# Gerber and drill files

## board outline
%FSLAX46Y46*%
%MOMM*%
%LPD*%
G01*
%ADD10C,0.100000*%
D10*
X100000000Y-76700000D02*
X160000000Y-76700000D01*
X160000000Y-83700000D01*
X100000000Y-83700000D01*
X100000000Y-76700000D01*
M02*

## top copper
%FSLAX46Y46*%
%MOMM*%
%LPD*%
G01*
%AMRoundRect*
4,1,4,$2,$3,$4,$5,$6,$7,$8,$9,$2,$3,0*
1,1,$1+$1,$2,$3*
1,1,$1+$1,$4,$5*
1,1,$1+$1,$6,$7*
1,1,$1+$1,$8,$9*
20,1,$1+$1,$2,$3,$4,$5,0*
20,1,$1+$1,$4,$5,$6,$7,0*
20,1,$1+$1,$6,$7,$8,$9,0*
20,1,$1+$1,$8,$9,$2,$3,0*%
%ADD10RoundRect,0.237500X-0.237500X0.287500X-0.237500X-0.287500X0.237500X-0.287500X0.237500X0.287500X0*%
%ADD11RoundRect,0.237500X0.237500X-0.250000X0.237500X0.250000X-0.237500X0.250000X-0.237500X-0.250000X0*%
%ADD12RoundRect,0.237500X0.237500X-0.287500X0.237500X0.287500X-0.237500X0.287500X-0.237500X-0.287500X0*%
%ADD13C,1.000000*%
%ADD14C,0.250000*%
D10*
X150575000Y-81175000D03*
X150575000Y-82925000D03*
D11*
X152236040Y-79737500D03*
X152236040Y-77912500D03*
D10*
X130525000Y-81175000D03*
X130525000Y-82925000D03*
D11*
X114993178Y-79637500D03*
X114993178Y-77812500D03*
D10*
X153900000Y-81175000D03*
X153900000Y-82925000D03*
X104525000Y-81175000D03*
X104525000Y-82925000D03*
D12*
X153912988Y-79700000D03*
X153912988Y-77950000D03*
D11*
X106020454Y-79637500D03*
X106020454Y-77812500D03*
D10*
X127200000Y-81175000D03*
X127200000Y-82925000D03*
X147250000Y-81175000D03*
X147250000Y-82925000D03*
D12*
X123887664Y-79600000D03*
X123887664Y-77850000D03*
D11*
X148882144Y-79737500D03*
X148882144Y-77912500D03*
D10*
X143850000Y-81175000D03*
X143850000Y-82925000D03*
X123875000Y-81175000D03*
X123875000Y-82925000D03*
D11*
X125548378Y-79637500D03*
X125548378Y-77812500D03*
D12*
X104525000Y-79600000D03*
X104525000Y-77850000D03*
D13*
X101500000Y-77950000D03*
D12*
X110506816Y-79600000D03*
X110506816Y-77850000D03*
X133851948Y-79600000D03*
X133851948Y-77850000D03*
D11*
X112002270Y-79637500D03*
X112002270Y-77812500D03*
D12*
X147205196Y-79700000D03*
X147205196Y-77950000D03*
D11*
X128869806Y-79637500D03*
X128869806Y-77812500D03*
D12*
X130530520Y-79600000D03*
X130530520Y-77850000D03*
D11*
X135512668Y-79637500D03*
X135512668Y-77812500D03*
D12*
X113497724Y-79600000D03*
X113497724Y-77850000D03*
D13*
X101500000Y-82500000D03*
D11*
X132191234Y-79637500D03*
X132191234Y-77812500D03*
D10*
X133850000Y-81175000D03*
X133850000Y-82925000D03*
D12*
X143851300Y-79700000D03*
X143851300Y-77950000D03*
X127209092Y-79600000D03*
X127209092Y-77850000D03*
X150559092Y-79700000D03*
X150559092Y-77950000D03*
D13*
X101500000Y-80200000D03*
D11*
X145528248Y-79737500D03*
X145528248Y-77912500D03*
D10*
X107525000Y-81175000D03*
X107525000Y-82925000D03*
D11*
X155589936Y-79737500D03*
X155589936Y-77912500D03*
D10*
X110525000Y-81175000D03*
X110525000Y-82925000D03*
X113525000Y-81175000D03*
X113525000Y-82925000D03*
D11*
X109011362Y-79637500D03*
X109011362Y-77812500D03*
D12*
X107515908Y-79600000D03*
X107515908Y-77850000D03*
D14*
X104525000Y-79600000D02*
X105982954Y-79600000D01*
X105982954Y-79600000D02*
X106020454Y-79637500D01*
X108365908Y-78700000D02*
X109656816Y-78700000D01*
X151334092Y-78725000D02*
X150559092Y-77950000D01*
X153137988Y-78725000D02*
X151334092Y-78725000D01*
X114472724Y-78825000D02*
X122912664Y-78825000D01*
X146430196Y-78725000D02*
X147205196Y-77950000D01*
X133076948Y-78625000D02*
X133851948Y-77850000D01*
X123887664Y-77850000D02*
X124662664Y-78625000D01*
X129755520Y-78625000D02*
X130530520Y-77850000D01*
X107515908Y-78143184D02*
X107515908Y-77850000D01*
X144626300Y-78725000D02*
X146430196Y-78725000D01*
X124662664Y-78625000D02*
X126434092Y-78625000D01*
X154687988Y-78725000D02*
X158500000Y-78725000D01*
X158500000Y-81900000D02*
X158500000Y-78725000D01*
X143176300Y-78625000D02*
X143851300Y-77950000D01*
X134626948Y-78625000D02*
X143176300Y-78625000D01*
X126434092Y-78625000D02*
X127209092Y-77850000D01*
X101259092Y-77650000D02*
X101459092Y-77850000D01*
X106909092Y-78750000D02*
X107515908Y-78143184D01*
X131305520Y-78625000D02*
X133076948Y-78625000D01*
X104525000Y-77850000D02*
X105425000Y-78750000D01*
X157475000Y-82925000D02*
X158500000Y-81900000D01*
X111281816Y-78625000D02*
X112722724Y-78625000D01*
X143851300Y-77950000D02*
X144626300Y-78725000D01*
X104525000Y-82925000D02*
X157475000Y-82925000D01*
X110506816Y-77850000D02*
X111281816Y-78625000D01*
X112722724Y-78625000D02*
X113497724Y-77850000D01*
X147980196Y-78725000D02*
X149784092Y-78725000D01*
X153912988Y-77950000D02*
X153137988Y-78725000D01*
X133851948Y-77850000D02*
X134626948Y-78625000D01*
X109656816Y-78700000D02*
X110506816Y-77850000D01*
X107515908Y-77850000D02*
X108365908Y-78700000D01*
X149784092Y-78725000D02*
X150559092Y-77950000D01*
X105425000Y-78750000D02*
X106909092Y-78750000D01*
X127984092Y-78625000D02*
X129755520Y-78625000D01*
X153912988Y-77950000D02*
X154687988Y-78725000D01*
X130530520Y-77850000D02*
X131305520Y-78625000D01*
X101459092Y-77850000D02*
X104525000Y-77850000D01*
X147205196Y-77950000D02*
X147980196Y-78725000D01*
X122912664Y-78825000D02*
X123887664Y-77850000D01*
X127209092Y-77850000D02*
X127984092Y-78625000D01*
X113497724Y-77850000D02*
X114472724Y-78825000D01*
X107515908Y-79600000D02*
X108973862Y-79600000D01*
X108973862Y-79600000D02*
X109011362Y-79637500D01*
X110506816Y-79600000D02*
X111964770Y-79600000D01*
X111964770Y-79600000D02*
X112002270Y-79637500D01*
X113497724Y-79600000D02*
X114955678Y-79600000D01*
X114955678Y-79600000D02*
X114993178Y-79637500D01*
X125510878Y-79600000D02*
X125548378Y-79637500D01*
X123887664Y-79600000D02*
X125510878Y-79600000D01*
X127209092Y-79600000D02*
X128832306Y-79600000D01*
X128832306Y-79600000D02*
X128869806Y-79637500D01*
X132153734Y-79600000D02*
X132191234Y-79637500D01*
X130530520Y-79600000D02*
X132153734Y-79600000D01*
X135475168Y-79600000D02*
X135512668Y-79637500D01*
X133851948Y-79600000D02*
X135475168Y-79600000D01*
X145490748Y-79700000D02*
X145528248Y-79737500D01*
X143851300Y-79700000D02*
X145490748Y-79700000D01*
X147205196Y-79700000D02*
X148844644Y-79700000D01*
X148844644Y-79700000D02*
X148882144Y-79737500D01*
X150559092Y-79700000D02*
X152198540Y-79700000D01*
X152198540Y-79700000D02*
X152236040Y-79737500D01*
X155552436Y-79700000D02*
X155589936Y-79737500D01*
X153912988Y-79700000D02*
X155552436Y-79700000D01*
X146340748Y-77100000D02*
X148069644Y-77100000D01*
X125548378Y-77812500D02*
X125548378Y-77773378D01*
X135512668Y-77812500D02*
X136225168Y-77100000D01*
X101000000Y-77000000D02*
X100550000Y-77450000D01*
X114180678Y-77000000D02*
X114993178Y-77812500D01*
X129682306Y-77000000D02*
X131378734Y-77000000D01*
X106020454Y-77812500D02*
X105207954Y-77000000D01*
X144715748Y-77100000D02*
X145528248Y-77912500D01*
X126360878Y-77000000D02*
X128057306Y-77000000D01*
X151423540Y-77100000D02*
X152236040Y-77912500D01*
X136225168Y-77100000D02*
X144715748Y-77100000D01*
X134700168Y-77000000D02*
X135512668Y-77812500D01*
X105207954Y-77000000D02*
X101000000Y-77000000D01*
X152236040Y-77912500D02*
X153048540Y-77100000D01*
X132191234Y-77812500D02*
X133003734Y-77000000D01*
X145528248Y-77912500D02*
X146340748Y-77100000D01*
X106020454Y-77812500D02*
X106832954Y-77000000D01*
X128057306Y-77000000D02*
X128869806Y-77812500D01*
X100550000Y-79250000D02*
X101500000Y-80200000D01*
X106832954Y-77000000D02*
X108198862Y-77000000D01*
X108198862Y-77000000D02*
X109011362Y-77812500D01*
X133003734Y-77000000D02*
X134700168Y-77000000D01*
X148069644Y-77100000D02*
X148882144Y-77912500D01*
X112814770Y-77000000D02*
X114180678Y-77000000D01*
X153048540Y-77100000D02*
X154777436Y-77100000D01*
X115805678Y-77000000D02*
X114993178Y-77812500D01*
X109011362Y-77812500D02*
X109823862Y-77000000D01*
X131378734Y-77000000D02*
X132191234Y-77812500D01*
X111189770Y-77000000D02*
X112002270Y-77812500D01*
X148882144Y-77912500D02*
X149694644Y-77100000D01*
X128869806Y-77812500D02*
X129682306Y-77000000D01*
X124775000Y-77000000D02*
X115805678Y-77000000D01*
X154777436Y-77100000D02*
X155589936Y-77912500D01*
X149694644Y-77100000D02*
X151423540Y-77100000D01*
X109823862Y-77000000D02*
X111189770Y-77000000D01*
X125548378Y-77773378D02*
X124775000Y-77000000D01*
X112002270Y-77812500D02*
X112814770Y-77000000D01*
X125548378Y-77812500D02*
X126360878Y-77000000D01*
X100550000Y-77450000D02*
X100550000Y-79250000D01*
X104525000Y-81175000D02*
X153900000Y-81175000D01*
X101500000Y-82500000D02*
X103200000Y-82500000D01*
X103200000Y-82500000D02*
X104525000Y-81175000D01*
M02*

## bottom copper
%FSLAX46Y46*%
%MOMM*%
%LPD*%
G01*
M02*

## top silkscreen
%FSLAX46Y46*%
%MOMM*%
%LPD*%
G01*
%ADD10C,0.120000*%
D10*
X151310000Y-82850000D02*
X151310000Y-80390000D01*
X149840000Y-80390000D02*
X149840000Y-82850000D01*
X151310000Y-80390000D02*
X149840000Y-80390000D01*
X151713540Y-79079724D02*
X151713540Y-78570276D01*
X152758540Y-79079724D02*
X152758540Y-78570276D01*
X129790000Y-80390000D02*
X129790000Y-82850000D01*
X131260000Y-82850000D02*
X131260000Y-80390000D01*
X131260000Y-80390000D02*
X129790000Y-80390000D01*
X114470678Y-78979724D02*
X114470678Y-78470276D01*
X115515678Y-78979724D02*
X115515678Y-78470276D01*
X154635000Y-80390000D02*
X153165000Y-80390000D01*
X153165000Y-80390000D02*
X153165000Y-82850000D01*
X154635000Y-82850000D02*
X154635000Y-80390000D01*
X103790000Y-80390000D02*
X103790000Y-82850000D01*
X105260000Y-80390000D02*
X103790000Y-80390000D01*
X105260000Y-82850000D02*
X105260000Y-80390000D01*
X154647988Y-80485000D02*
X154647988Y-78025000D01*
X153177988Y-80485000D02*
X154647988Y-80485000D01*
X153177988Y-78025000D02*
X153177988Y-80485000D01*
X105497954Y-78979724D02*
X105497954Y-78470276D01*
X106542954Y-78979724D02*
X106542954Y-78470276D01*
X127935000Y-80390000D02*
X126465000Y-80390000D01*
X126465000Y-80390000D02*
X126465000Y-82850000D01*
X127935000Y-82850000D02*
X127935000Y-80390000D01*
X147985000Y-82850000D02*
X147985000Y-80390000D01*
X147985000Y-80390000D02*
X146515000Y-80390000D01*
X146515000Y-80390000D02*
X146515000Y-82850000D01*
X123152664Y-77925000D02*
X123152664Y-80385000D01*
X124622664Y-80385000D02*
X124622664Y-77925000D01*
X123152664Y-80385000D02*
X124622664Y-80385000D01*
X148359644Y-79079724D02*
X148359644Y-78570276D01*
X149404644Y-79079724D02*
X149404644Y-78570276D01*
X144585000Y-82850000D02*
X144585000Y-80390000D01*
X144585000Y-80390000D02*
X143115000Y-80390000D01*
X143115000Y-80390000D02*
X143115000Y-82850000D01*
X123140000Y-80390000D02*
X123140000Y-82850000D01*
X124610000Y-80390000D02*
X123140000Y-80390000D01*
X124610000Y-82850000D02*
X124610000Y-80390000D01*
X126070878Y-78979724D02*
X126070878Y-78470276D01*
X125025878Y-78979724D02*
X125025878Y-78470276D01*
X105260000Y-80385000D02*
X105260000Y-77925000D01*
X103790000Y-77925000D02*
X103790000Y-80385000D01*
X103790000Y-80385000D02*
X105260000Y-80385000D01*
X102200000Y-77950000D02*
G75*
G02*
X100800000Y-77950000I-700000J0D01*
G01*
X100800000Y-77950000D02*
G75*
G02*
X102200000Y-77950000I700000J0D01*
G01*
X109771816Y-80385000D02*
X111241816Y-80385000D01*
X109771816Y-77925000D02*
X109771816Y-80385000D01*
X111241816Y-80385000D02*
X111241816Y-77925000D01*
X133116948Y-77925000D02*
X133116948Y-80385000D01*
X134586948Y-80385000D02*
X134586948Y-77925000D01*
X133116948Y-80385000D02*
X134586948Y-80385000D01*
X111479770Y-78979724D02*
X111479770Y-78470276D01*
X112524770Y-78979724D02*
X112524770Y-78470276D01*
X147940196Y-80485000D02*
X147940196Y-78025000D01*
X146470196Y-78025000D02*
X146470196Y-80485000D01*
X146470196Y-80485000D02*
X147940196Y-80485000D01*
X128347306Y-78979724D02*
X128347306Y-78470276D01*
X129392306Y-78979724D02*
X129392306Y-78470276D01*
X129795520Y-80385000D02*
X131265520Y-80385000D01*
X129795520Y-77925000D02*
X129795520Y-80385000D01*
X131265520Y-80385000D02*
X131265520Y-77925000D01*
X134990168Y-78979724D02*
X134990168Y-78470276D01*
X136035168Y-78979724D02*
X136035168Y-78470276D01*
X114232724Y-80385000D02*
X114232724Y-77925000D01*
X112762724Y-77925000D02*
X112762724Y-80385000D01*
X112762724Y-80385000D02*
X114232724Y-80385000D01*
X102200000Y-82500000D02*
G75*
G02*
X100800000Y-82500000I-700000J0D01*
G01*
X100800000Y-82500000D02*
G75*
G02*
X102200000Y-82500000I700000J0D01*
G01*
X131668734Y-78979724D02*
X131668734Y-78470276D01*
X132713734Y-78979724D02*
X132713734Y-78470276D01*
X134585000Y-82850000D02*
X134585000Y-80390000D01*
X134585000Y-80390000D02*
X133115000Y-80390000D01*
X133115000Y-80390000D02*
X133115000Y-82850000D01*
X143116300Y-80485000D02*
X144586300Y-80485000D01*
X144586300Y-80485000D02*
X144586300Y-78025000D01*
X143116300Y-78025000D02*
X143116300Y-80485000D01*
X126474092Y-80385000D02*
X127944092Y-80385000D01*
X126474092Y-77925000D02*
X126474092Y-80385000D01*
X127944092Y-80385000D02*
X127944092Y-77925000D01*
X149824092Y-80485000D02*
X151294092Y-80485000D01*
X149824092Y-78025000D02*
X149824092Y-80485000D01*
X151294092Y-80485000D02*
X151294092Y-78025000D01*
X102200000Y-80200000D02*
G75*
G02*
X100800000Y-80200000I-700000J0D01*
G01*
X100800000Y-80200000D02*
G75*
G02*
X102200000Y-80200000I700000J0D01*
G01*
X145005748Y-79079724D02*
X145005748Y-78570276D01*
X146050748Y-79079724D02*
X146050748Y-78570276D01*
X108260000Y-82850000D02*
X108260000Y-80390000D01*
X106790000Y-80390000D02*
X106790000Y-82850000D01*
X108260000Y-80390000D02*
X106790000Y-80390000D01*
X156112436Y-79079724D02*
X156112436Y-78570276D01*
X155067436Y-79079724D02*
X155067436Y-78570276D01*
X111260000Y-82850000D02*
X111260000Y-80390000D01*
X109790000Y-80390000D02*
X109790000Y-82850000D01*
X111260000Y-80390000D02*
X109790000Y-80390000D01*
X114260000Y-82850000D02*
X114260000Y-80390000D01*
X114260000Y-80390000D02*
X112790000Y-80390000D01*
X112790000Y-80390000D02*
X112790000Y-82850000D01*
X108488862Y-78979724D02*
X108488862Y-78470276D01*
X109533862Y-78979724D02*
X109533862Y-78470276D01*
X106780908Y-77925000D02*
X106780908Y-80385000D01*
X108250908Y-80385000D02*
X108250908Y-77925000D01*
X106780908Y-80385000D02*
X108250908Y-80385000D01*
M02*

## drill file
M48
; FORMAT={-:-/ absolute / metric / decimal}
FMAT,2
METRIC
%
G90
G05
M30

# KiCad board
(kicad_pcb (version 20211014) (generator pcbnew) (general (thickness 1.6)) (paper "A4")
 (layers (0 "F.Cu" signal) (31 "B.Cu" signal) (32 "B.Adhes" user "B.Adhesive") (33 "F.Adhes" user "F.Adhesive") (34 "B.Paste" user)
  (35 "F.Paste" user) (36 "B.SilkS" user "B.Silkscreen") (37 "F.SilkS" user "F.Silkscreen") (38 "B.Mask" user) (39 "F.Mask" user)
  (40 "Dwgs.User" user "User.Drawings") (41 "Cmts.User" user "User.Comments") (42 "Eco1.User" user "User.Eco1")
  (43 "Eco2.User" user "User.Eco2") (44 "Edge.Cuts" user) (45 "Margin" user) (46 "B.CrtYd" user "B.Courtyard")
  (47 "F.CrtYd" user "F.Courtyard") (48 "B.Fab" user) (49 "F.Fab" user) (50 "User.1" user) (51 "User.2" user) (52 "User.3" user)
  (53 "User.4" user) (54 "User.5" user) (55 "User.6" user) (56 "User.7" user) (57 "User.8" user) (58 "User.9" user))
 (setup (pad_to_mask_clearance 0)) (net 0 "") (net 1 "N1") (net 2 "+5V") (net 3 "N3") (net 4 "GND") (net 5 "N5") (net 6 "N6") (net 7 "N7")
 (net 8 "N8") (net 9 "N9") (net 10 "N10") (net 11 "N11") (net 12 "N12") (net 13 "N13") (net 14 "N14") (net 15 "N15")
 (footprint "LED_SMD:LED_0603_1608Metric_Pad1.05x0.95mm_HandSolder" (layer "F.Cu") (at 150.575 82.05 -90)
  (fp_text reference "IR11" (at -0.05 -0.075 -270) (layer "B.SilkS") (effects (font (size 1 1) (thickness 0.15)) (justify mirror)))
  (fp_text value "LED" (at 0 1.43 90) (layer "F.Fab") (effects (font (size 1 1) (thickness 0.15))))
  (fp_line (start 0.8 -0.735) (end -1.66 -0.735) (layer "F.SilkS") (width 0.12))
  (fp_line (start -1.66 0.735) (end 0.8 0.735) (layer "F.SilkS") (width 0.12))
  (fp_line (start -1.66 -0.735) (end -1.66 0.735) (layer "F.SilkS") (width 0.12))
  (pad "1" smd roundrect (at -0.875 0 270) (size 1.05 0.95) (layers "F.Cu" "F.Paste" "F.Mask") (roundrect_rratio 0.25) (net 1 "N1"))
  (pad "2" smd roundrect (at 0.875 0 270) (size 1.05 0.95) (layers "F.Cu" "F.Paste" "F.Mask") (roundrect_rratio 0.25) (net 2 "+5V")))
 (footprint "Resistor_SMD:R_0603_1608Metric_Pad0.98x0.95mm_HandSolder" (layer "F.Cu") (at 152.23604 78.825 90)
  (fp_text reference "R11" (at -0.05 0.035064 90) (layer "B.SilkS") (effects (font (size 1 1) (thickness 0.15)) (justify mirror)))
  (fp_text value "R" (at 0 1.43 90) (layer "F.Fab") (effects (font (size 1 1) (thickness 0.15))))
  (fp_line (start -0.254724 -0.5225) (end 0.254724 -0.5225) (layer "F.SilkS") (width 0.12))
  (fp_line (start -0.254724 0.5225) (end 0.254724 0.5225) (layer "F.SilkS") (width 0.12))
  (pad "1" smd roundrect (at -0.9125 0 90) (size 0.975 0.95) (layers "F.Cu" "F.Paste" "F.Mask") (roundrect_rratio 0.25) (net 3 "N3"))
  (pad "2" smd roundrect (at 0.9125 0 90) (size 0.975 0.95) (layers "F.Cu" "F.Paste" "F.Mask") (roundrect_rratio 0.25) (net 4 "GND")))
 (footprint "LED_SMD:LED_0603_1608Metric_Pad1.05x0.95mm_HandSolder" (layer "F.Cu") (at 130.525 82.05 -90)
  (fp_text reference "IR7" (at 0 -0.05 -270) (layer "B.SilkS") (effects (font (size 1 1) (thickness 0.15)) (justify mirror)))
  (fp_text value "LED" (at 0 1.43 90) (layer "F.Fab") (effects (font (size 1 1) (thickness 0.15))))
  (fp_line (start -1.66 0.735) (end 0.8 0.735) (layer "F.SilkS") (width 0.12))
  (fp_line (start 0.8 -0.735) (end -1.66 -0.735) (layer "F.SilkS") (width 0.12))
  (fp_line (start -1.66 -0.735) (end -1.66 0.735) (layer "F.SilkS") (width 0.12))
  (pad "1" smd roundrect (at -0.875 0 270) (size 1.05 0.95) (layers "F.Cu" "F.Paste" "F.Mask") (roundrect_rratio 0.25) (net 1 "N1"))
  (pad "2" smd roundrect (at 0.875 0 270) (size 1.05 0.95) (layers "F.Cu" "F.Paste" "F.Mask") (roundrect_rratio 0.25) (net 2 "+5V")))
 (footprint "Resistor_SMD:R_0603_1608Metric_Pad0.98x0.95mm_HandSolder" (layer "F.Cu") (at 114.993178 78.725 90)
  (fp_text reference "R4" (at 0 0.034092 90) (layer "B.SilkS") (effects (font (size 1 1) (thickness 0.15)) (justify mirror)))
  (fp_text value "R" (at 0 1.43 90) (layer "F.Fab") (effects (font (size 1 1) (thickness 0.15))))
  (fp_line (start -0.254724 -0.5225) (end 0.254724 -0.5225) (layer "F.SilkS") (width 0.12))
  (fp_line (start -0.254724 0.5225) (end 0.254724 0.5225) (layer "F.SilkS") (width 0.12))
  (pad "1" smd roundrect (at -0.9125 0 90) (size 0.975 0.95) (layers "F.Cu" "F.Paste" "F.Mask") (roundrect_rratio 0.25) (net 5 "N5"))
  (pad "2" smd roundrect (at 0.9125 0 90) (size 0.975 0.95) (layers "F.Cu" "F.Paste" "F.Mask") (roundrect_rratio 0.25) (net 4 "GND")))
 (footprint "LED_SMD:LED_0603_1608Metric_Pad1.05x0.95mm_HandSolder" (layer "F.Cu") (at 153.9 82.05 -90)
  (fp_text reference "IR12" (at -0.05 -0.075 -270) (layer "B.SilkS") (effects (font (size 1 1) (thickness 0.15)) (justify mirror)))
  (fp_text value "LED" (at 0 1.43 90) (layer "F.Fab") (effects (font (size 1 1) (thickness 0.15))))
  (fp_line (start -1.66 -0.735) (end -1.66 0.735) (layer "F.SilkS") (width 0.12))
  (fp_line (start -1.66 0.735) (end 0.8 0.735) (layer "F.SilkS") (width 0.12))
  (fp_line (start 0.8 -0.735) (end -1.66 -0.735) (layer "F.SilkS") (width 0.12))
  (pad "1" smd roundrect (at -0.875 0 270) (size 1.05 0.95) (layers "F.Cu" "F.Paste" "F.Mask") (roundrect_rratio 0.25) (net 1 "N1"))
  (pad "2" smd roundrect (at 0.875 0 270) (size 1.05 0.95) (layers "F.Cu" "F.Paste" "F.Mask") (roundrect_rratio 0.25) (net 2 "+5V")))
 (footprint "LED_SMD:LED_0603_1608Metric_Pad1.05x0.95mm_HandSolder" (layer "F.Cu") (at 104.525 82.05 -90)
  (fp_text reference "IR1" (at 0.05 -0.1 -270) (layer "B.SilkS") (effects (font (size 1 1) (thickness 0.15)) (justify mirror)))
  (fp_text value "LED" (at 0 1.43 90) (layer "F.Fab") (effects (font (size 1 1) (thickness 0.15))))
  (fp_line (start -1.66 0.735) (end 0.8 0.735) (layer "F.SilkS") (width 0.12))
  (fp_line (start -1.66 -0.735) (end -1.66 0.735) (layer "F.SilkS") (width 0.12))
  (fp_line (start 0.8 -0.735) (end -1.66 -0.735) (layer "F.SilkS") (width 0.12))
  (pad "1" smd roundrect (at -0.875 0 270) (size 1.05 0.95) (layers "F.Cu" "F.Paste" "F.Mask") (roundrect_rratio 0.25) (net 1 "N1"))
  (pad "2" smd roundrect (at 0.875 0 270) (size 1.05 0.95) (layers "F.Cu" "F.Paste" "F.Mask") (roundrect_rratio 0.25) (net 2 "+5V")))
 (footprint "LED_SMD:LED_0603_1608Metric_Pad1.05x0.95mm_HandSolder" (layer "F.Cu") (at 153.912988 78.825 90)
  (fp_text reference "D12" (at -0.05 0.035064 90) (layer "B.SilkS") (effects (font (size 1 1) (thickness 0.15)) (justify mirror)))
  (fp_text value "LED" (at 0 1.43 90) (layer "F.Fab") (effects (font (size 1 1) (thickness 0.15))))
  (fp_line (start -1.66 0.735) (end 0.8 0.735) (layer "F.SilkS") (width 0.12))
  (fp_line (start -1.66 -0.735) (end -1.66 0.735) (layer "F.SilkS") (width 0.12))
  (fp_line (start 0.8 -0.735) (end -1.66 -0.735) (layer "F.SilkS") (width 0.12))
  (pad "1" smd roundrect (at -0.875 0 90) (size 1.05 0.95) (layers "F.Cu" "F.Paste" "F.Mask") (roundrect_rratio 0.25) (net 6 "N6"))
  (pad "2" smd roundrect (at 0.875 0 90) (size 1.05 0.95) (layers "F.Cu" "F.Paste" "F.Mask") (roundrect_rratio 0.25) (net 2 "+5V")))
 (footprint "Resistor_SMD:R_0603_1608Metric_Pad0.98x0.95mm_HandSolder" (layer "F.Cu") (at 106.020454 78.725 90)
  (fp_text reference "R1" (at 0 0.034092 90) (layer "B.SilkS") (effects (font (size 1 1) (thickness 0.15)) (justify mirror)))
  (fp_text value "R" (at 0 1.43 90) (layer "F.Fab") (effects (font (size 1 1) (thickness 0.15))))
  (fp_line (start -0.254724 -0.5225) (end 0.254724 -0.5225) (layer "F.SilkS") (width 0.12))
  (fp_line (start -0.254724 0.5225) (end 0.254724 0.5225) (layer "F.SilkS") (width 0.12))
  (pad "1" smd roundrect (at -0.9125 0 90) (size 0.975 0.95) (layers "F.Cu" "F.Paste" "F.Mask") (roundrect_rratio 0.25) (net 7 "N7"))
  (pad "2" smd roundrect (at 0.9125 0 90) (size 0.975 0.95) (layers "F.Cu" "F.Paste" "F.Mask") (roundrect_rratio 0.25) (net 4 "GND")))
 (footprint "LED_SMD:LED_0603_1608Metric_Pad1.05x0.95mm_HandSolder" (layer "F.Cu") (at 127.2 82.05 -90)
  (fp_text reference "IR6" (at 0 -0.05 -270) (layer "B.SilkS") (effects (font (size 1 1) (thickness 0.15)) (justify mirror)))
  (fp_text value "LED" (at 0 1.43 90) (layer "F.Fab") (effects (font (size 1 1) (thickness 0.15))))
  (fp_line (start -1.66 -0.735) (end -1.66 0.735) (layer "F.SilkS") (width 0.12))
  (fp_line (start -1.66 0.735) (end 0.8 0.735) (layer "F.SilkS") (width 0.12))
  (fp_line (start 0.8 -0.735) (end -1.66 -0.735) (layer "F.SilkS") (width 0.12))
  (pad "1" smd roundrect (at -0.875 0 270) (size 1.05 0.95) (layers "F.Cu" "F.Paste" "F.Mask") (roundrect_rratio 0.25) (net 1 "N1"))
  (pad "2" smd roundrect (at 0.875 0 270) (size 1.05 0.95) (layers "F.Cu" "F.Paste" "F.Mask") (roundrect_rratio 0.25) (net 2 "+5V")))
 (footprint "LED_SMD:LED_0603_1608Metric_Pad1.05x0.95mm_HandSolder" (layer "F.Cu") (at 147.25 82.05 -90)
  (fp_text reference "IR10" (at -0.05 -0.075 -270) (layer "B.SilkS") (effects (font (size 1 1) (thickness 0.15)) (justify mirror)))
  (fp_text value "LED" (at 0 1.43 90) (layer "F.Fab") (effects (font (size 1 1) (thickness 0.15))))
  (fp_line (start 0.8 -0.735) (end -1.66 -0.735) (layer "F.SilkS") (width 0.12))
  (fp_line (start -1.66 -0.735) (end -1.66 0.735) (layer "F.SilkS") (width 0.12))
  (fp_line (start -1.66 0.735) (end 0.8 0.735) (layer "F.SilkS") (width 0.12))
  (pad "1" smd roundrect (at -0.875 0 270) (size 1.05 0.95) (layers "F.Cu" "F.Paste" "F.Mask") (roundrect_rratio 0.25) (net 1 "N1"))
  (pad "2" smd roundrect (at 0.875 0 270) (size 1.05 0.95) (layers "F.Cu" "F.Paste" "F.Mask") (roundrect_rratio 0.25) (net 2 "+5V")))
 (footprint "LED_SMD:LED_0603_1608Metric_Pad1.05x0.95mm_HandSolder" (layer "F.Cu") (at 123.887664 78.725 90)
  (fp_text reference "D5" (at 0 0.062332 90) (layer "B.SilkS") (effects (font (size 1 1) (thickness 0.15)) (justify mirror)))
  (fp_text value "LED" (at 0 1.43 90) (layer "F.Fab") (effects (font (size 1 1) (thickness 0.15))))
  (fp_line (start 0.8 -0.735) (end -1.66 -0.735) (layer "F.SilkS") (width 0.12))
  (fp_line (start -1.66 0.735) (end 0.8 0.735) (layer "F.SilkS") (width 0.12))
  (fp_line (start -1.66 -0.735) (end -1.66 0.735) (layer "F.SilkS") (width 0.12))
  (pad "1" smd roundrect (at -0.875 0 90) (size 1.05 0.95) (layers "F.Cu" "F.Paste" "F.Mask") (roundrect_rratio 0.25) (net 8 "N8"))
  (pad "2" smd roundrect (at 0.875 0 90) (size 1.05 0.95) (layers "F.Cu" "F.Paste" "F.Mask") (roundrect_rratio 0.25) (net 2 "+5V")))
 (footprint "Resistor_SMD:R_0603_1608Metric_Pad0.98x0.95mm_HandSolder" (layer "F.Cu") (at 148.882144 78.825 90)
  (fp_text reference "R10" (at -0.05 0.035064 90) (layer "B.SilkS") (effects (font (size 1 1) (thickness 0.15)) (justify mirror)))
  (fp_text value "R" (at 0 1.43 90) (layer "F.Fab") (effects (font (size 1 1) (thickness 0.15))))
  (fp_line (start -0.254724 -0.5225) (end 0.254724 -0.5225) (layer "F.SilkS") (width 0.12))
  (fp_line (start -0.254724 0.5225) (end 0.254724 0.5225) (layer "F.SilkS") (width 0.12))
  (pad "1" smd roundrect (at -0.9125 0 90) (size 0.975 0.95) (layers "F.Cu" "F.Paste" "F.Mask") (roundrect_rratio 0.25) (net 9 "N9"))
  (pad "2" smd roundrect (at 0.9125 0 90) (size 0.975 0.95) (layers "F.Cu" "F.Paste" "F.Mask") (roundrect_rratio 0.25) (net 4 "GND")))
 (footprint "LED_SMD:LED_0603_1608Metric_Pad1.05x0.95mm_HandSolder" (layer "F.Cu") (at 143.85 82.05 -90)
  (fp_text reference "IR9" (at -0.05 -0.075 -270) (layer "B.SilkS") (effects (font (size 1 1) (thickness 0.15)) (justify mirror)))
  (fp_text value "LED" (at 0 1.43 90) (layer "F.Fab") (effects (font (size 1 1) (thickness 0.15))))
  (fp_line (start 0.8 -0.735) (end -1.66 -0.735) (layer "F.SilkS") (width 0.12))
  (fp_line (start -1.66 -0.735) (end -1.66 0.735) (layer "F.SilkS") (width 0.12))
  (fp_line (start -1.66 0.735) (end 0.8 0.735) (layer "F.SilkS") (width 0.12))
  (pad "1" smd roundrect (at -0.875 0 270) (size 1.05 0.95) (layers "F.Cu" "F.Paste" "F.Mask") (roundrect_rratio 0.25) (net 1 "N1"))
  (pad "2" smd roundrect (at 0.875 0 270) (size 1.05 0.95) (layers "F.Cu" "F.Paste" "F.Mask") (roundrect_rratio 0.25) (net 2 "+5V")))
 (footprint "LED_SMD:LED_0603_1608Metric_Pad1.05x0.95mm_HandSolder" (layer "F.Cu") (at 123.875 82.05 -90)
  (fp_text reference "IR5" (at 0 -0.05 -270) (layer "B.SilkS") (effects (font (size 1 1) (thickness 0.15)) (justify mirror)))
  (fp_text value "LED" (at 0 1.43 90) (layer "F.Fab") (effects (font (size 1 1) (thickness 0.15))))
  (fp_line (start -1.66 0.735) (end 0.8 0.735) (layer "F.SilkS") (width 0.12))
  (fp_line (start -1.66 -0.735) (end -1.66 0.735) (layer "F.SilkS") (width 0.12))
  (fp_line (start 0.8 -0.735) (end -1.66 -0.735) (layer "F.SilkS") (width 0.12))
  (pad "1" smd roundrect (at -0.875 0 270) (size 1.05 0.95) (layers "F.Cu" "F.Paste" "F.Mask") (roundrect_rratio 0.25) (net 1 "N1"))
  (pad "2" smd roundrect (at 0.875 0 270) (size 1.05 0.95) (layers "F.Cu" "F.Paste" "F.Mask") (roundrect_rratio 0.25) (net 2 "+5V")))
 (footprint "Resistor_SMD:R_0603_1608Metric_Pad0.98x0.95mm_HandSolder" (layer "F.Cu") (at 125.548378 78.725 90)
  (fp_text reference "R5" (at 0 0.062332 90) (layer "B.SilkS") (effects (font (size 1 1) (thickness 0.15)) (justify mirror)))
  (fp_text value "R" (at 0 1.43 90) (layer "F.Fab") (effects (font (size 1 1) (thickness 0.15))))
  (fp_line (start -0.254724 0.5225) (end 0.254724 0.5225) (layer "F.SilkS") (width 0.12))
  (fp_line (start -0.254724 -0.5225) (end 0.254724 -0.5225) (layer "F.SilkS") (width 0.12))
  (pad "1" smd roundrect (at -0.9125 0 90) (size 0.975 0.95) (layers "F.Cu" "F.Paste" "F.Mask") (roundrect_rratio 0.25) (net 8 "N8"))
  (pad "2" smd roundrect (at 0.9125 0 90) (size 0.975 0.95) (layers "F.Cu" "F.Paste" "F.Mask") (roundrect_rratio 0.25) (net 4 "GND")))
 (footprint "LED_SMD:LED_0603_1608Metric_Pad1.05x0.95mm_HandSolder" (layer "F.Cu") (at 104.525 78.725 90)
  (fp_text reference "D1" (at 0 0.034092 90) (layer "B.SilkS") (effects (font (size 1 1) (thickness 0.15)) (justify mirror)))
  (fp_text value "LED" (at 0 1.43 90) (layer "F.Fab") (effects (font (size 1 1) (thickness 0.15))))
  (fp_line (start -1.66 0.735) (end 0.8 0.735) (layer "F.SilkS") (width 0.12))
  (fp_line (start 0.8 -0.735) (end -1.66 -0.735) (layer "F.SilkS") (width 0.12))
  (fp_line (start -1.66 -0.735) (end -1.66 0.735) (layer "F.SilkS") (width 0.12))
  (pad "1" smd roundrect (at -0.875 0 90) (size 1.05 0.95) (layers "F.Cu" "F.Paste" "F.Mask") (roundrect_rratio 0.25) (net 7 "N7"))
  (pad "2" smd roundrect (at 0.875 0 90) (size 1.05 0.95) (layers "F.Cu" "F.Paste" "F.Mask") (roundrect_rratio 0.25) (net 2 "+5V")))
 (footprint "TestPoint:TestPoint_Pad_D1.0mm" (layer "F.Cu") (at 101.5 77.95)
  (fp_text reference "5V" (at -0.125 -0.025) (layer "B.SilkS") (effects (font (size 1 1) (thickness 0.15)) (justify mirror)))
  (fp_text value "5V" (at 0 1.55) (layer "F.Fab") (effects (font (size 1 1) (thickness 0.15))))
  (fp_circle (center 0 0) (end 0 0.7) (layer "F.SilkS") (width 0.12) (fill none))
  (pad "1" smd circle (at 0 0) (size 1 1) (layers "F.Cu" "F.Mask") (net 2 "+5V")))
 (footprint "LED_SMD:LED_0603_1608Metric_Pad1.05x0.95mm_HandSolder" (layer "F.Cu") (at 110.506816 78.725 90)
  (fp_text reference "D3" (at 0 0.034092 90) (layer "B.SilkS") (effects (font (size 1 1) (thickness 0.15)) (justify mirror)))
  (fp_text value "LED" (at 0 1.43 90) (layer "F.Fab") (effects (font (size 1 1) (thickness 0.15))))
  (fp_line (start -1.66 -0.735) (end -1.66 0.735) (layer "F.SilkS") (width 0.12))
  (fp_line (start 0.8 -0.735) (end -1.66 -0.735) (layer "F.SilkS") (width 0.12))
  (fp_line (start -1.66 0.735) (end 0.8 0.735) (layer "F.SilkS") (width 0.12))
  (pad "1" smd roundrect (at -0.875 0 90) (size 1.05 0.95) (layers "F.Cu" "F.Paste" "F.Mask") (roundrect_rratio 0.25) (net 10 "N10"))
  (pad "2" smd roundrect (at 0.875 0 90) (size 1.05 0.95) (layers "F.Cu" "F.Paste" "F.Mask") (roundrect_rratio 0.25) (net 2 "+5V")))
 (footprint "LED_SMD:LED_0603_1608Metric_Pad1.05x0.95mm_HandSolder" (layer "F.Cu") (at 133.851948 78.725 90)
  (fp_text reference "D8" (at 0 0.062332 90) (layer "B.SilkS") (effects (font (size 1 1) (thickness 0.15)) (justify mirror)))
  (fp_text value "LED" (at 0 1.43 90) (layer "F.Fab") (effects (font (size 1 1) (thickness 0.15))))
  (fp_line (start 0.8 -0.735) (end -1.66 -0.735) (layer "F.SilkS") (width 0.12))
  (fp_line (start -1.66 0.735) (end 0.8 0.735) (layer "F.SilkS") (width 0.12))
  (fp_line (start -1.66 -0.735) (end -1.66 0.735) (layer "F.SilkS") (width 0.12))
  (pad "1" smd roundrect (at -0.875 0 90) (size 1.05 0.95) (layers "F.Cu" "F.Paste" "F.Mask") (roundrect_rratio 0.25) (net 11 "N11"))
  (pad "2" smd roundrect (at 0.875 0 90) (size 1.05 0.95) (layers "F.Cu" "F.Paste" "F.Mask") (roundrect_rratio 0.25) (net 2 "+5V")))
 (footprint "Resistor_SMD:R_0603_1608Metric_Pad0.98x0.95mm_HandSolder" (layer "F.Cu") (at 112.00227 78.725 90)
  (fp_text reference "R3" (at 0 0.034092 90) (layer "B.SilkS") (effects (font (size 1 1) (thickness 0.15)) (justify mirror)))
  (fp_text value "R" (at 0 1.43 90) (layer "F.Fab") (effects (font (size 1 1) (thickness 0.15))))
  (fp_line (start -0.254724 -0.5225) (end 0.254724 -0.5225) (layer "F.SilkS") (width 0.12))
  (fp_line (start -0.254724 0.5225) (end 0.254724 0.5225) (layer "F.SilkS") (width 0.12))
  (pad "1" smd roundrect (at -0.9125 0 90) (size 0.975 0.95) (layers "F.Cu" "F.Paste" "F.Mask") (roundrect_rratio 0.25) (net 10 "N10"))
  (pad "2" smd roundrect (at 0.9125 0 90) (size 0.975 0.95) (layers "F.Cu" "F.Paste" "F.Mask") (roundrect_rratio 0.25) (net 4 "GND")))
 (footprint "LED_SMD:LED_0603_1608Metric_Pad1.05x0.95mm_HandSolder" (layer "F.Cu") (at 147.205196 78.825 90)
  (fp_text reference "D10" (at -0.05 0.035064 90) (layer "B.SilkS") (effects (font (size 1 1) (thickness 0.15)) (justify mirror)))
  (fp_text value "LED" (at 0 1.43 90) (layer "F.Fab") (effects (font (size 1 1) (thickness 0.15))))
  (fp_line (start -1.66 0.735) (end 0.8 0.735) (layer "F.SilkS") (width 0.12))
  (fp_line (start 0.8 -0.735) (end -1.66 -0.735) (layer "F.SilkS") (width 0.12))
  (fp_line (start -1.66 -0.735) (end -1.66 0.735) (layer "F.SilkS") (width 0.12))
  (pad "1" smd roundrect (at -0.875 0 90) (size 1.05 0.95) (layers "F.Cu" "F.Paste" "F.Mask") (roundrect_rratio 0.25) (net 9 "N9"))
  (pad "2" smd roundrect (at 0.875 0 90) (size 1.05 0.95) (layers "F.Cu" "F.Paste" "F.Mask") (roundrect_rratio 0.25) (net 2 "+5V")))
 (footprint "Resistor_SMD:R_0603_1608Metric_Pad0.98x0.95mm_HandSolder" (layer "F.Cu") (at 128.869806 78.725 90)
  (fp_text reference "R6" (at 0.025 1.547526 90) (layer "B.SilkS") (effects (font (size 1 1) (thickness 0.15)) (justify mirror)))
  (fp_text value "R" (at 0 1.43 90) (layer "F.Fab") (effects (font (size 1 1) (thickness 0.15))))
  (fp_line (start -0.254724 -0.5225) (end 0.254724 -0.5225) (layer "F.SilkS") (width 0.12))
  (fp_line (start -0.254724 0.5225) (end 0.254724 0.5225) (layer "F.SilkS") (width 0.12))
  (pad "1" smd roundrect (at -0.9125 0 90) (size 0.975 0.95) (layers "F.Cu" "F.Paste" "F.Mask") (roundrect_rratio 0.25) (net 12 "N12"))
  (pad "2" smd roundrect (at 0.9125 0 90) (size 0.975 0.95) (layers "F.Cu" "F.Paste" "F.Mask") (roundrect_rratio 0.25) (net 4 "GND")))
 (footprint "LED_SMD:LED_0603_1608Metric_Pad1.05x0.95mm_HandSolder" (layer "F.Cu") (at 130.53052 78.725 90)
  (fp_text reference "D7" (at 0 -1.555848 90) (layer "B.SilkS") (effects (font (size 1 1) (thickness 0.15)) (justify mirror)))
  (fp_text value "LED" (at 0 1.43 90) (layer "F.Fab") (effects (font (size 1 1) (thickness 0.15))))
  (fp_line (start -1.66 -0.735) (end -1.66 0.735) (layer "F.SilkS") (width 0.12))
  (fp_line (start 0.8 -0.735) (end -1.66 -0.735) (layer "F.SilkS") (width 0.12))
  (fp_line (start -1.66 0.735) (end 0.8 0.735) (layer "F.SilkS") (width 0.12))
  (pad "1" smd roundrect (at -0.875 0 90) (size 1.05 0.95) (layers "F.Cu" "F.Paste" "F.Mask") (roundrect_rratio 0.25) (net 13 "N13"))
  (pad "2" smd roundrect (at 0.875 0 90) (size 1.05 0.95) (layers "F.Cu" "F.Paste" "F.Mask") (roundrect_rratio 0.25) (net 2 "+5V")))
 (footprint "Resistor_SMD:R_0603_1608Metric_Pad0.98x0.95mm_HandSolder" (layer "F.Cu") (at 135.512668 78.725 90)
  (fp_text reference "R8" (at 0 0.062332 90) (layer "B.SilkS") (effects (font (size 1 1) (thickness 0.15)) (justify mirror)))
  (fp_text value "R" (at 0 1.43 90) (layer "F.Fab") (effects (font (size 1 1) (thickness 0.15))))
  (fp_line (start -0.254724 -0.5225) (end 0.254724 -0.5225) (layer "F.SilkS") (width 0.12))
  (fp_line (start -0.254724 0.5225) (end 0.254724 0.5225) (layer "F.SilkS") (width 0.12))
  (pad "1" smd roundrect (at -0.9125 0 90) (size 0.975 0.95) (layers "F.Cu" "F.Paste" "F.Mask") (roundrect_rratio 0.25) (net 11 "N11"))
  (pad "2" smd roundrect (at 0.9125 0 90) (size 0.975 0.95) (layers "F.Cu" "F.Paste" "F.Mask") (roundrect_rratio 0.25) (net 4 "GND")))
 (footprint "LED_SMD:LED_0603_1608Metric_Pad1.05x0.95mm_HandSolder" (layer "F.Cu") (at 113.497724 78.725 90)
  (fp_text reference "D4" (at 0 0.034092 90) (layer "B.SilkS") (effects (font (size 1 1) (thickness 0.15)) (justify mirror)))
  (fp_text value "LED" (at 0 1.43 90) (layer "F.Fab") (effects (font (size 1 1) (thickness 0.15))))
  (fp_line (start -1.66 0.735) (end 0.8 0.735) (layer "F.SilkS") (width 0.12))
  (fp_line (start 0.8 -0.735) (end -1.66 -0.735) (layer "F.SilkS") (width 0.12))
  (fp_line (start -1.66 -0.735) (end -1.66 0.735) (layer "F.SilkS") (width 0.12))
  (pad "1" smd roundrect (at -0.875 0 90) (size 1.05 0.95) (layers "F.Cu" "F.Paste" "F.Mask") (roundrect_rratio 0.25) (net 5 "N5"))
  (pad "2" smd roundrect (at 0.875 0 90) (size 1.05 0.95) (layers "F.Cu" "F.Paste" "F.Mask") (roundrect_rratio 0.25) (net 2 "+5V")))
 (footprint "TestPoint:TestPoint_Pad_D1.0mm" (layer "F.Cu") (at 101.5 82.5)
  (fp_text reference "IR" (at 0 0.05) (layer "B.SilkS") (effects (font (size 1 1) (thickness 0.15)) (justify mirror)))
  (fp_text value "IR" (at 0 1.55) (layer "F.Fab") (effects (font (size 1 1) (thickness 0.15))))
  (fp_circle (center 0 0) (end 0 0.7) (layer "F.SilkS") (width 0.12) (fill none))
  (pad "1" smd circle (at 0 0) (size 1 1) (layers "F.Cu" "F.Mask") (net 1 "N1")))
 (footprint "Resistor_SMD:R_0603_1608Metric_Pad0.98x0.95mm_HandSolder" (layer "F.Cu") (at 132.191234 78.725 90)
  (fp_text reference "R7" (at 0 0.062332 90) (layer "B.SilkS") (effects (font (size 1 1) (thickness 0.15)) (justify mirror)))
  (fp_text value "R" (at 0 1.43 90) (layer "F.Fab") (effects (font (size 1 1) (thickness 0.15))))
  (fp_line (start -0.254724 -0.5225) (end 0.254724 -0.5225) (layer "F.SilkS") (width 0.12))
  (fp_line (start -0.254724 0.5225) (end 0.254724 0.5225) (layer "F.SilkS") (width 0.12))
  (pad "1" smd roundrect (at -0.9125 0 90) (size 0.975 0.95) (layers "F.Cu" "F.Paste" "F.Mask") (roundrect_rratio 0.25) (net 13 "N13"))
  (pad "2" smd roundrect (at 0.9125 0 90) (size 0.975 0.95) (layers "F.Cu" "F.Paste" "F.Mask") (roundrect_rratio 0.25) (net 4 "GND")))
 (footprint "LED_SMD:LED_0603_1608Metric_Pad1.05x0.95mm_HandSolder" (layer "F.Cu") (at 133.85 82.05 -90)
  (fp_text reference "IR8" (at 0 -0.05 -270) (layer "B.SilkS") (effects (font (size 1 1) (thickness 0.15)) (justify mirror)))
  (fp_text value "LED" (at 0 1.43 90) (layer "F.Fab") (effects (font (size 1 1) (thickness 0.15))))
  (fp_line (start 0.8 -0.735) (end -1.66 -0.735) (layer "F.SilkS") (width 0.12))
  (fp_line (start -1.66 -0.735) (end -1.66 0.735) (layer "F.SilkS") (width 0.12))
  (fp_line (start -1.66 0.735) (end 0.8 0.735) (layer "F.SilkS") (width 0.12))
  (pad "1" smd roundrect (at -0.875 0 270) (size 1.05 0.95) (layers "F.Cu" "F.Paste" "F.Mask") (roundrect_rratio 0.25) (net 1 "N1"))
  (pad "2" smd roundrect (at 0.875 0 270) (size 1.05 0.95) (layers "F.Cu" "F.Paste" "F.Mask") (roundrect_rratio 0.25) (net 2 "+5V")))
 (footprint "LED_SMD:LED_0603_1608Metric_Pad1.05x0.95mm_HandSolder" (layer "F.Cu") (at 143.8513 78.825 90)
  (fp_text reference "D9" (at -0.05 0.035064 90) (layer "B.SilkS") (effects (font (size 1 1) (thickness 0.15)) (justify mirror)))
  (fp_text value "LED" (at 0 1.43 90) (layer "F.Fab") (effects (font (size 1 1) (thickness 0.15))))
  (fp_line (start -1.66 -0.735) (end -1.66 0.735) (layer "F.SilkS") (width 0.12))
  (fp_line (start -1.66 0.735) (end 0.8 0.735) (layer "F.SilkS") (width 0.12))
  (fp_line (start 0.8 -0.735) (end -1.66 -0.735) (layer "F.SilkS") (width 0.12))
  (pad "1" smd roundrect (at -0.875 0 90) (size 1.05 0.95) (layers "F.Cu" "F.Paste" "F.Mask") (roundrect_rratio 0.25) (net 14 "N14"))
  (pad "2" smd roundrect (at 0.875 0 90) (size 1.05 0.95) (layers "F.Cu" "F.Paste" "F.Mask") (roundrect_rratio 0.25) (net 2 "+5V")))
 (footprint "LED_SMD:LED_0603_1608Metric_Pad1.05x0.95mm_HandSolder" (layer "F.Cu") (at 127.209092 78.725 90)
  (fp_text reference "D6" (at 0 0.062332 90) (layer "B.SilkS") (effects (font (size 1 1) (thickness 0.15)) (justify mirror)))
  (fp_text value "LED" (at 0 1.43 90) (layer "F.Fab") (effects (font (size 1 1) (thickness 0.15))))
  (fp_line (start -1.66 -0.735) (end -1.66 0.735) (layer "F.SilkS") (width 0.12))
  (fp_line (start 0.8 -0.735) (end -1.66 -0.735) (layer "F.SilkS") (width 0.12))
  (fp_line (start -1.66 0.735) (end 0.8 0.735) (layer "F.SilkS") (width 0.12))
  (pad "1" smd roundrect (at -0.875 0 90) (size 1.05 0.95) (layers "F.Cu" "F.Paste" "F.Mask") (roundrect_rratio 0.25) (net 12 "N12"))
  (pad "2" smd roundrect (at 0.875 0 90) (size 1.05 0.95) (layers "F.Cu" "F.Paste" "F.Mask") (roundrect_rratio 0.25) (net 2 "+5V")))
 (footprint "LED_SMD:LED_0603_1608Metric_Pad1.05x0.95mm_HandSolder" (layer "F.Cu") (at 150.559092 78.825 90)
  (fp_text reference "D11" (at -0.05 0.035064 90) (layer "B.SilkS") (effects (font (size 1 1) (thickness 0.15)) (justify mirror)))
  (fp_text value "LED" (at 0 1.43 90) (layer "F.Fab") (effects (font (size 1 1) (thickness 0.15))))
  (fp_line (start -1.66 -0.735) (end -1.66 0.735) (layer "F.SilkS") (width 0.12))
  (fp_line (start 0.8 -0.735) (end -1.66 -0.735) (layer "F.SilkS") (width 0.12))
  (fp_line (start -1.66 0.735) (end 0.8 0.735) (layer "F.SilkS") (width 0.12))
  (pad "1" smd roundrect (at -0.875 0 90) (size 1.05 0.95) (layers "F.Cu" "F.Paste" "F.Mask") (roundrect_rratio 0.25) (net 3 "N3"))
  (pad "2" smd roundrect (at 0.875 0 90) (size 1.05 0.95) (layers "F.Cu" "F.Paste" "F.Mask") (roundrect_rratio 0.25) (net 2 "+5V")))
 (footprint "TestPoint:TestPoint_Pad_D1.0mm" (layer "F.Cu") (at 101.5 80.2)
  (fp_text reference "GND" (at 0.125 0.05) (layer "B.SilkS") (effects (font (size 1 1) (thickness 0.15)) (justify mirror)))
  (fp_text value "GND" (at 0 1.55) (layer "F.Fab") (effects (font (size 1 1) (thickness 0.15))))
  (fp_circle (center 0 0) (end 0 0.7) (layer "F.SilkS") (width 0.12) (fill none))
  (pad "1" smd circle (at 0 0) (size 1 1) (layers "F.Cu" "F.Mask") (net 4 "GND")))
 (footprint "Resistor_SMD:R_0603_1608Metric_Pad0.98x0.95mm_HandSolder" (layer "F.Cu") (at 145.528248 78.825 90)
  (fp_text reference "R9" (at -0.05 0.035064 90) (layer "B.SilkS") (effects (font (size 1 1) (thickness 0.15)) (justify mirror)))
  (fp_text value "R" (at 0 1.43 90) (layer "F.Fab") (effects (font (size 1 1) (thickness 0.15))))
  (fp_line (start -0.254724 -0.5225) (end 0.254724 -0.5225) (layer "F.SilkS") (width 0.12))
  (fp_line (start -0.254724 0.5225) (end 0.254724 0.5225) (layer "F.SilkS") (width 0.12))
  (pad "1" smd roundrect (at -0.9125 0 90) (size 0.975 0.95) (layers "F.Cu" "F.Paste" "F.Mask") (roundrect_rratio 0.25) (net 14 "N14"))
  (pad "2" smd roundrect (at 0.9125 0 90) (size 0.975 0.95) (layers "F.Cu" "F.Paste" "F.Mask") (roundrect_rratio 0.25) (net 4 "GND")))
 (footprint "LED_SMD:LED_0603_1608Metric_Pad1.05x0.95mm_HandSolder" (layer "F.Cu") (at 107.525 82.05 -90)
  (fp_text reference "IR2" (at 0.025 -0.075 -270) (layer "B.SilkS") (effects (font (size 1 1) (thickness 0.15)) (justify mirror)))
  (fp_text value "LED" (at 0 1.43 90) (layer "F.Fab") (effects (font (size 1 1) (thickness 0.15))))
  (fp_line (start 0.8 -0.735) (end -1.66 -0.735) (layer "F.SilkS") (width 0.12))
  (fp_line (start -1.66 0.735) (end 0.8 0.735) (layer "F.SilkS") (width 0.12))
  (fp_line (start -1.66 -0.735) (end -1.66 0.735) (layer "F.SilkS") (width 0.12))
  (pad "1" smd roundrect (at -0.875 0 270) (size 1.05 0.95) (layers "F.Cu" "F.Paste" "F.Mask") (roundrect_rratio 0.25) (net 1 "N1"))
  (pad "2" smd roundrect (at 0.875 0 270) (size 1.05 0.95) (layers "F.Cu" "F.Paste" "F.Mask") (roundrect_rratio 0.25) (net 2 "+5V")))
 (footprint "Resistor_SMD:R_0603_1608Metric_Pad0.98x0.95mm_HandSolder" (layer "F.Cu") (at 155.589936 78.825 90)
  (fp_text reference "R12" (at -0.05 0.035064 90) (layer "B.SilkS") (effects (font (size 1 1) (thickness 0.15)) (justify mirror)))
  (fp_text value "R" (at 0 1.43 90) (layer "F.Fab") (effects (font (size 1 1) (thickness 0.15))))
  (fp_line (start -0.254724 0.5225) (end 0.254724 0.5225) (layer "F.SilkS") (width 0.12))
  (fp_line (start -0.254724 -0.5225) (end 0.254724 -0.5225) (layer "F.SilkS") (width 0.12))
  (pad "1" smd roundrect (at -0.9125 0 90) (size 0.975 0.95) (layers "F.Cu" "F.Paste" "F.Mask") (roundrect_rratio 0.25) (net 6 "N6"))
  (pad "2" smd roundrect (at 0.9125 0 90) (size 0.975 0.95) (layers "F.Cu" "F.Paste" "F.Mask") (roundrect_rratio 0.25) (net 4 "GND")))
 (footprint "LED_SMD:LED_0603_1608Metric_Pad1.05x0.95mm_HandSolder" (layer "F.Cu") (at 110.525 82.05 -90)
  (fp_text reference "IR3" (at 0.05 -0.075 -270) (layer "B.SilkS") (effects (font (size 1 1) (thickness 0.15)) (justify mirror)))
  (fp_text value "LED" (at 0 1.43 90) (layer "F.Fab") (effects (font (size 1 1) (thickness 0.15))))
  (fp_line (start 0.8 -0.735) (end -1.66 -0.735) (layer "F.SilkS") (width 0.12))
  (fp_line (start -1.66 0.735) (end 0.8 0.735) (layer "F.SilkS") (width 0.12))
  (fp_line (start -1.66 -0.735) (end -1.66 0.735) (layer "F.SilkS") (width 0.12))
  (pad "1" smd roundrect (at -0.875 0 270) (size 1.05 0.95) (layers "F.Cu" "F.Paste" "F.Mask") (roundrect_rratio 0.25) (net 1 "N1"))
  (pad "2" smd roundrect (at 0.875 0 270) (size 1.05 0.95) (layers "F.Cu" "F.Paste" "F.Mask") (roundrect_rratio 0.25) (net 2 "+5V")))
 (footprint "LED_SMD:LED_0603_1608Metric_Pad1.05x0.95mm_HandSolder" (layer "F.Cu") (at 113.525 82.05 -90)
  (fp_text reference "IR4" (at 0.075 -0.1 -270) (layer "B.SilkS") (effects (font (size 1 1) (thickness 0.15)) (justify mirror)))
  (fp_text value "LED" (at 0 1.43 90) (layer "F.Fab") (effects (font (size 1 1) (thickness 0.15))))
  (fp_line (start 0.8 -0.735) (end -1.66 -0.735) (layer "F.SilkS") (width 0.12))
  (fp_line (start -1.66 -0.735) (end -1.66 0.735) (layer "F.SilkS") (width 0.12))
  (fp_line (start -1.66 0.735) (end 0.8 0.735) (layer "F.SilkS") (width 0.12))
  (pad "1" smd roundrect (at -0.875 0 270) (size 1.05 0.95) (layers "F.Cu" "F.Paste" "F.Mask") (roundrect_rratio 0.25) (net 1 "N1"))
  (pad "2" smd roundrect (at 0.875 0 270) (size 1.05 0.95) (layers "F.Cu" "F.Paste" "F.Mask") (roundrect_rratio 0.25) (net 2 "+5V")))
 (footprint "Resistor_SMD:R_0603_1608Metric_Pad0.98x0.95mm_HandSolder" (layer "F.Cu") (at 109.011362 78.725 90)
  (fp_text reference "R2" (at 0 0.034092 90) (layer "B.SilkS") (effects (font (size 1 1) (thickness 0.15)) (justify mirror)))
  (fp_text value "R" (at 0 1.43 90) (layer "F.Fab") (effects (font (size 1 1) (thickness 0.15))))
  (fp_line (start -0.254724 -0.5225) (end 0.254724 -0.5225) (layer "F.SilkS") (width 0.12))
  (fp_line (start -0.254724 0.5225) (end 0.254724 0.5225) (layer "F.SilkS") (width 0.12))
  (pad "1" smd roundrect (at -0.9125 0 90) (size 0.975 0.95) (layers "F.Cu" "F.Paste" "F.Mask") (roundrect_rratio 0.25) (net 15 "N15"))
  (pad "2" smd roundrect (at 0.9125 0 90) (size 0.975 0.95) (layers "F.Cu" "F.Paste" "F.Mask") (roundrect_rratio 0.25) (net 4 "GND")))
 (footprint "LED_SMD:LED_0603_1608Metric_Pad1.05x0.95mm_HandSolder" (layer "F.Cu") (at 107.515908 78.725 90)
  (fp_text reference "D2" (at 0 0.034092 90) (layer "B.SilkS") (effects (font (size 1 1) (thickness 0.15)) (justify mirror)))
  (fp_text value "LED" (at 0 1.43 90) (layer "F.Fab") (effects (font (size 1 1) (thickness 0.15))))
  (fp_line (start 0.8 -0.735) (end -1.66 -0.735) (layer "F.SilkS") (width 0.12))
  (fp_line (start -1.66 0.735) (end 0.8 0.735) (layer "F.SilkS") (width 0.12))
  (fp_line (start -1.66 -0.735) (end -1.66 0.735) (layer "F.SilkS") (width 0.12))
  (pad "1" smd roundrect (at -0.875 0 90) (size 1.05 0.95) (layers "F.Cu" "F.Paste" "F.Mask") (roundrect_rratio 0.25) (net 15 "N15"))
  (pad "2" smd roundrect (at 0.875 0 90) (size 1.05 0.95) (layers "F.Cu" "F.Paste" "F.Mask") (roundrect_rratio 0.25) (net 2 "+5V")))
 (gr_rect (start 100 76.7) (end 160 83.7) (layer "Edge.Cuts") (width 0.1) (fill none))
 (segment (start 104.525 79.6) (end 105.982954 79.6) (width 0.25) (layer "F.Cu") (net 7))
 (segment (start 105.982954 79.6) (end 106.020454 79.6375) (width 0.25) (layer "F.Cu") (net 7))
 (segment (start 108.365908 78.7) (end 109.656816 78.7) (width 0.25) (layer "F.Cu") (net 2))
 (segment (start 151.334092 78.725) (end 150.559092 77.95) (width 0.25) (layer "F.Cu") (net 2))
 (segment (start 153.137988 78.725) (end 151.334092 78.725) (width 0.25) (layer "F.Cu") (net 2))
 (segment (start 114.472724 78.825) (end 122.912664 78.825) (width 0.25) (layer "F.Cu") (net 2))
 (segment (start 146.430196 78.725) (end 147.205196 77.95) (width 0.25) (layer "F.Cu") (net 2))
 (segment (start 133.076948 78.625) (end 133.851948 77.85) (width 0.25) (layer "F.Cu") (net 2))
 (segment (start 123.887664 77.85) (end 124.662664 78.625) (width 0.25) (layer "F.Cu") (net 2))
 (segment (start 129.75552 78.625) (end 130.53052 77.85) (width 0.25) (layer "F.Cu") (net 2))
 (segment (start 107.515908 78.143184) (end 107.515908 77.85) (width 0.25) (layer "F.Cu") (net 2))
 (segment (start 144.6263 78.725) (end 146.430196 78.725) (width 0.25) (layer "F.Cu") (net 2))
 (segment (start 124.662664 78.625) (end 126.434092 78.625) (width 0.25) (layer "F.Cu") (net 2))
 (segment (start 154.687988 78.725) (end 158.5 78.725) (width 0.25) (layer "F.Cu") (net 2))
 (segment (start 158.5 81.9) (end 158.5 78.725) (width 0.25) (layer "F.Cu") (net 2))
 (segment (start 143.1763 78.625) (end 143.8513 77.95) (width 0.25) (layer "F.Cu") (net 2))
 (segment (start 134.626948 78.625) (end 143.1763 78.625) (width 0.25) (layer "F.Cu") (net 2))
 (segment (start 126.434092 78.625) (end 127.209092 77.85) (width 0.25) (layer "F.Cu") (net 2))
 (segment (start 101.259092 77.65) (end 101.459092 77.85) (width 0.25) (layer "F.Cu") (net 2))
 (segment (start 106.909092 78.75) (end 107.515908 78.143184) (width 0.25) (layer "F.Cu") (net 2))
 (segment (start 131.30552 78.625) (end 133.076948 78.625) (width 0.25) (layer "F.Cu") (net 2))
 (segment (start 104.525 77.85) (end 105.425 78.75) (width 0.25) (layer "F.Cu") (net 2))
 (segment (start 157.475 82.925) (end 158.5 81.9) (width 0.25) (layer "F.Cu") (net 2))
 (segment (start 111.281816 78.625) (end 112.722724 78.625) (width 0.25) (layer "F.Cu") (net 2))
 (segment (start 143.8513 77.95) (end 144.6263 78.725) (width 0.25) (layer "F.Cu") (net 2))
 (segment (start 104.525 82.925) (end 157.475 82.925) (width 0.25) (layer "F.Cu") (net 2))
 (segment (start 110.506816 77.85) (end 111.281816 78.625) (width 0.25) (layer "F.Cu") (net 2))
 (segment (start 112.722724 78.625) (end 113.497724 77.85) (width 0.25) (layer "F.Cu") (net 2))
 (segment (start 147.980196 78.725) (end 149.784092 78.725) (width 0.25) (layer "F.Cu") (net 2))
 (segment (start 153.912988 77.95) (end 153.137988 78.725) (width 0.25) (layer "F.Cu") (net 2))
 (segment (start 133.851948 77.85) (end 134.626948 78.625) (width 0.25) (layer "F.Cu") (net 2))
 (segment (start 109.656816 78.7) (end 110.506816 77.85) (width 0.25) (layer "F.Cu") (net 2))
 (segment (start 107.515908 77.85) (end 108.365908 78.7) (width 0.25) (layer "F.Cu") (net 2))
 (segment (start 149.784092 78.725) (end 150.559092 77.95) (width 0.25) (layer "F.Cu") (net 2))
 (segment (start 105.425 78.75) (end 106.909092 78.75) (width 0.25) (layer "F.Cu") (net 2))
 (segment (start 127.984092 78.625) (end 129.75552 78.625) (width 0.25) (layer "F.Cu") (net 2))
 (segment (start 153.912988 77.95) (end 154.687988 78.725) (width 0.25) (layer "F.Cu") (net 2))
 (segment (start 130.53052 77.85) (end 131.30552 78.625) (width 0.25) (layer "F.Cu") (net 2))
 (segment (start 101.459092 77.85) (end 104.525 77.85) (width 0.25) (layer "F.Cu") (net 2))
 (segment (start 147.205196 77.95) (end 147.980196 78.725) (width 0.25) (layer "F.Cu") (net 2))
 (segment (start 122.912664 78.825) (end 123.887664 77.85) (width 0.25) (layer "F.Cu") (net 2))
 (segment (start 127.209092 77.85) (end 127.984092 78.625) (width 0.25) (layer "F.Cu") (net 2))
 (segment (start 113.497724 77.85) (end 114.472724 78.825) (width 0.25) (layer "F.Cu") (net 2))
 (segment (start 107.515908 79.6) (end 108.973862 79.6) (width 0.25) (layer "F.Cu") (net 15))
 (segment (start 108.973862 79.6) (end 109.011362 79.6375) (width 0.25) (layer "F.Cu") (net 15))
 (segment (start 110.506816 79.6) (end 111.96477 79.6) (width 0.25) (layer "F.Cu") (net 10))
 (segment (start 111.96477 79.6) (end 112.00227 79.6375) (width 0.25) (layer "F.Cu") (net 10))
 (segment (start 113.497724 79.6) (end 114.955678 79.6) (width 0.25) (layer "F.Cu") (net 5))
 (segment (start 114.955678 79.6) (end 114.993178 79.6375) (width 0.25) (layer "F.Cu") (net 5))
 (segment (start 125.510878 79.6) (end 125.548378 79.6375) (width 0.25) (layer "F.Cu") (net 8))
 (segment (start 123.887664 79.6) (end 125.510878 79.6) (width 0.25) (layer "F.Cu") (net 8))
 (segment (start 127.209092 79.6) (end 128.832306 79.6) (width 0.25) (layer "F.Cu") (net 12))
 (segment (start 128.832306 79.6) (end 128.869806 79.6375) (width 0.25) (layer "F.Cu") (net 12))
 (segment (start 132.153734 79.6) (end 132.191234 79.6375) (width 0.25) (layer "F.Cu") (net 13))
 (segment (start 130.53052 79.6) (end 132.153734 79.6) (width 0.25) (layer "F.Cu") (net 13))
 (segment (start 135.475168 79.6) (end 135.512668 79.6375) (width 0.25) (layer "F.Cu") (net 11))
 (segment (start 133.851948 79.6) (end 135.475168 79.6) (width 0.25) (layer "F.Cu") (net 11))
 (segment (start 145.490748 79.7) (end 145.528248 79.7375) (width 0.25) (layer "F.Cu") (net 14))
 (segment (start 143.8513 79.7) (end 145.490748 79.7) (width 0.25) (layer "F.Cu") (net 14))
 (segment (start 147.205196 79.7) (end 148.844644 79.7) (width 0.25) (layer "F.Cu") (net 9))
 (segment (start 148.844644 79.7) (end 148.882144 79.7375) (width 0.25) (layer "F.Cu") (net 9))
 (segment (start 150.559092 79.7) (end 152.19854 79.7) (width 0.25) (layer "F.Cu") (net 3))
 (segment (start 152.19854 79.7) (end 152.23604 79.7375) (width 0.25) (layer "F.Cu") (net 3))
 (segment (start 155.552436 79.7) (end 155.589936 79.7375) (width 0.25) (layer "F.Cu") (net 6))
 (segment (start 153.912988 79.7) (end 155.552436 79.7) (width 0.25) (layer "F.Cu") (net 6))
 (segment (start 146.340748 77.1) (end 148.069644 77.1) (width 0.25) (layer "F.Cu") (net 4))
 (segment (start 125.548378 77.8125) (end 125.548378 77.773378) (width 0.25) (layer "F.Cu") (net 4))
 (segment (start 135.512668 77.8125) (end 136.225168 77.1) (width 0.25) (layer "F.Cu") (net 4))
 (segment (start 101 77) (end 100.55 77.45) (width 0.25) (layer "F.Cu") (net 4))
 (segment (start 114.180678 77) (end 114.993178 77.8125) (width 0.25) (layer "F.Cu") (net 4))
 (segment (start 129.682306 77) (end 131.378734 77) (width 0.25) (layer "F.Cu") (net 4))
 (segment (start 106.020454 77.8125) (end 105.207954 77) (width 0.25) (layer "F.Cu") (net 4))
 (segment (start 144.715748 77.1) (end 145.528248 77.9125) (width 0.25) (layer "F.Cu") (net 4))
 (segment (start 126.360878 77) (end 128.057306 77) (width 0.25) (layer "F.Cu") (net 4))
 (segment (start 151.42354 77.1) (end 152.23604 77.9125) (width 0.25) (layer "F.Cu") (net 4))
 (segment (start 136.225168 77.1) (end 144.715748 77.1) (width 0.25) (layer "F.Cu") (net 4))
 (segment (start 134.700168 77) (end 135.512668 77.8125) (width 0.25) (layer "F.Cu") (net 4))
 (segment (start 105.207954 77) (end 101 77) (width 0.25) (layer "F.Cu") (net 4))
 (segment (start 152.23604 77.9125) (end 153.04854 77.1) (width 0.25) (layer "F.Cu") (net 4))
 (segment (start 132.191234 77.8125) (end 133.003734 77) (width 0.25) (layer "F.Cu") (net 4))
 (segment (start 145.528248 77.9125) (end 146.340748 77.1) (width 0.25) (layer "F.Cu") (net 4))
 (segment (start 106.020454 77.8125) (end 106.832954 77) (width 0.25) (layer "F.Cu") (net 4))
 (segment (start 128.057306 77) (end 128.869806 77.8125) (width 0.25) (layer "F.Cu") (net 4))
 (segment (start 100.55 79.25) (end 101.5 80.2) (width 0.25) (layer "F.Cu") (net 4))
 (segment (start 106.832954 77) (end 108.198862 77) (width 0.25) (layer "F.Cu") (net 4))
 (segment (start 108.198862 77) (end 109.011362 77.8125) (width 0.25) (layer "F.Cu") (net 4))
 (segment (start 133.003734 77) (end 134.700168 77) (width 0.25) (layer "F.Cu") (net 4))
 (segment (start 148.069644 77.1) (end 148.882144 77.9125) (width 0.25) (layer "F.Cu") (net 4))
 (segment (start 112.81477 77) (end 114.180678 77) (width 0.25) (layer "F.Cu") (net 4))
 (segment (start 153.04854 77.1) (end 154.777436 77.1) (width 0.25) (layer "F.Cu") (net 4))
 (segment (start 115.805678 77) (end 114.993178 77.8125) (width 0.25) (layer "F.Cu") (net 4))
 (segment (start 109.011362 77.8125) (end 109.823862 77) (width 0.25) (layer "F.Cu") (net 4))
 (segment (start 131.378734 77) (end 132.191234 77.8125) (width 0.25) (layer "F.Cu") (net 4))
 (segment (start 111.18977 77) (end 112.00227 77.8125) (width 0.25) (layer "F.Cu") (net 4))
 (segment (start 148.882144 77.9125) (end 149.694644 77.1) (width 0.25) (layer "F.Cu") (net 4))
 (segment (start 128.869806 77.8125) (end 129.682306 77) (width 0.25) (layer "F.Cu") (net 4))
 (segment (start 124.775 77) (end 115.805678 77) (width 0.25) (layer "F.Cu") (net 4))
 (segment (start 154.777436 77.1) (end 155.589936 77.9125) (width 0.25) (layer "F.Cu") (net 4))
 (segment (start 149.694644 77.1) (end 151.42354 77.1) (width 0.25) (layer "F.Cu") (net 4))
 (segment (start 109.823862 77) (end 111.18977 77) (width 0.25) (layer "F.Cu") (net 4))
 (segment (start 125.548378 77.773378) (end 124.775 77) (width 0.25) (layer "F.Cu") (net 4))
 (segment (start 112.00227 77.8125) (end 112.81477 77) (width 0.25) (layer "F.Cu") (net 4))
 (segment (start 125.548378 77.8125) (end 126.360878 77) (width 0.25) (layer "F.Cu") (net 4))
 (segment (start 100.55 77.45) (end 100.55 79.25) (width 0.25) (layer "F.Cu") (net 4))
 (segment (start 104.525 81.175) (end 153.9 81.175) (width 0.25) (layer "F.Cu") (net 1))
 (segment (start 101.5 82.5) (end 103.2 82.5) (width 0.25) (layer "F.Cu") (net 1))
 (segment (start 103.2 82.5) (end 104.525 81.175) (width 0.25) (layer "F.Cu") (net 1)))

